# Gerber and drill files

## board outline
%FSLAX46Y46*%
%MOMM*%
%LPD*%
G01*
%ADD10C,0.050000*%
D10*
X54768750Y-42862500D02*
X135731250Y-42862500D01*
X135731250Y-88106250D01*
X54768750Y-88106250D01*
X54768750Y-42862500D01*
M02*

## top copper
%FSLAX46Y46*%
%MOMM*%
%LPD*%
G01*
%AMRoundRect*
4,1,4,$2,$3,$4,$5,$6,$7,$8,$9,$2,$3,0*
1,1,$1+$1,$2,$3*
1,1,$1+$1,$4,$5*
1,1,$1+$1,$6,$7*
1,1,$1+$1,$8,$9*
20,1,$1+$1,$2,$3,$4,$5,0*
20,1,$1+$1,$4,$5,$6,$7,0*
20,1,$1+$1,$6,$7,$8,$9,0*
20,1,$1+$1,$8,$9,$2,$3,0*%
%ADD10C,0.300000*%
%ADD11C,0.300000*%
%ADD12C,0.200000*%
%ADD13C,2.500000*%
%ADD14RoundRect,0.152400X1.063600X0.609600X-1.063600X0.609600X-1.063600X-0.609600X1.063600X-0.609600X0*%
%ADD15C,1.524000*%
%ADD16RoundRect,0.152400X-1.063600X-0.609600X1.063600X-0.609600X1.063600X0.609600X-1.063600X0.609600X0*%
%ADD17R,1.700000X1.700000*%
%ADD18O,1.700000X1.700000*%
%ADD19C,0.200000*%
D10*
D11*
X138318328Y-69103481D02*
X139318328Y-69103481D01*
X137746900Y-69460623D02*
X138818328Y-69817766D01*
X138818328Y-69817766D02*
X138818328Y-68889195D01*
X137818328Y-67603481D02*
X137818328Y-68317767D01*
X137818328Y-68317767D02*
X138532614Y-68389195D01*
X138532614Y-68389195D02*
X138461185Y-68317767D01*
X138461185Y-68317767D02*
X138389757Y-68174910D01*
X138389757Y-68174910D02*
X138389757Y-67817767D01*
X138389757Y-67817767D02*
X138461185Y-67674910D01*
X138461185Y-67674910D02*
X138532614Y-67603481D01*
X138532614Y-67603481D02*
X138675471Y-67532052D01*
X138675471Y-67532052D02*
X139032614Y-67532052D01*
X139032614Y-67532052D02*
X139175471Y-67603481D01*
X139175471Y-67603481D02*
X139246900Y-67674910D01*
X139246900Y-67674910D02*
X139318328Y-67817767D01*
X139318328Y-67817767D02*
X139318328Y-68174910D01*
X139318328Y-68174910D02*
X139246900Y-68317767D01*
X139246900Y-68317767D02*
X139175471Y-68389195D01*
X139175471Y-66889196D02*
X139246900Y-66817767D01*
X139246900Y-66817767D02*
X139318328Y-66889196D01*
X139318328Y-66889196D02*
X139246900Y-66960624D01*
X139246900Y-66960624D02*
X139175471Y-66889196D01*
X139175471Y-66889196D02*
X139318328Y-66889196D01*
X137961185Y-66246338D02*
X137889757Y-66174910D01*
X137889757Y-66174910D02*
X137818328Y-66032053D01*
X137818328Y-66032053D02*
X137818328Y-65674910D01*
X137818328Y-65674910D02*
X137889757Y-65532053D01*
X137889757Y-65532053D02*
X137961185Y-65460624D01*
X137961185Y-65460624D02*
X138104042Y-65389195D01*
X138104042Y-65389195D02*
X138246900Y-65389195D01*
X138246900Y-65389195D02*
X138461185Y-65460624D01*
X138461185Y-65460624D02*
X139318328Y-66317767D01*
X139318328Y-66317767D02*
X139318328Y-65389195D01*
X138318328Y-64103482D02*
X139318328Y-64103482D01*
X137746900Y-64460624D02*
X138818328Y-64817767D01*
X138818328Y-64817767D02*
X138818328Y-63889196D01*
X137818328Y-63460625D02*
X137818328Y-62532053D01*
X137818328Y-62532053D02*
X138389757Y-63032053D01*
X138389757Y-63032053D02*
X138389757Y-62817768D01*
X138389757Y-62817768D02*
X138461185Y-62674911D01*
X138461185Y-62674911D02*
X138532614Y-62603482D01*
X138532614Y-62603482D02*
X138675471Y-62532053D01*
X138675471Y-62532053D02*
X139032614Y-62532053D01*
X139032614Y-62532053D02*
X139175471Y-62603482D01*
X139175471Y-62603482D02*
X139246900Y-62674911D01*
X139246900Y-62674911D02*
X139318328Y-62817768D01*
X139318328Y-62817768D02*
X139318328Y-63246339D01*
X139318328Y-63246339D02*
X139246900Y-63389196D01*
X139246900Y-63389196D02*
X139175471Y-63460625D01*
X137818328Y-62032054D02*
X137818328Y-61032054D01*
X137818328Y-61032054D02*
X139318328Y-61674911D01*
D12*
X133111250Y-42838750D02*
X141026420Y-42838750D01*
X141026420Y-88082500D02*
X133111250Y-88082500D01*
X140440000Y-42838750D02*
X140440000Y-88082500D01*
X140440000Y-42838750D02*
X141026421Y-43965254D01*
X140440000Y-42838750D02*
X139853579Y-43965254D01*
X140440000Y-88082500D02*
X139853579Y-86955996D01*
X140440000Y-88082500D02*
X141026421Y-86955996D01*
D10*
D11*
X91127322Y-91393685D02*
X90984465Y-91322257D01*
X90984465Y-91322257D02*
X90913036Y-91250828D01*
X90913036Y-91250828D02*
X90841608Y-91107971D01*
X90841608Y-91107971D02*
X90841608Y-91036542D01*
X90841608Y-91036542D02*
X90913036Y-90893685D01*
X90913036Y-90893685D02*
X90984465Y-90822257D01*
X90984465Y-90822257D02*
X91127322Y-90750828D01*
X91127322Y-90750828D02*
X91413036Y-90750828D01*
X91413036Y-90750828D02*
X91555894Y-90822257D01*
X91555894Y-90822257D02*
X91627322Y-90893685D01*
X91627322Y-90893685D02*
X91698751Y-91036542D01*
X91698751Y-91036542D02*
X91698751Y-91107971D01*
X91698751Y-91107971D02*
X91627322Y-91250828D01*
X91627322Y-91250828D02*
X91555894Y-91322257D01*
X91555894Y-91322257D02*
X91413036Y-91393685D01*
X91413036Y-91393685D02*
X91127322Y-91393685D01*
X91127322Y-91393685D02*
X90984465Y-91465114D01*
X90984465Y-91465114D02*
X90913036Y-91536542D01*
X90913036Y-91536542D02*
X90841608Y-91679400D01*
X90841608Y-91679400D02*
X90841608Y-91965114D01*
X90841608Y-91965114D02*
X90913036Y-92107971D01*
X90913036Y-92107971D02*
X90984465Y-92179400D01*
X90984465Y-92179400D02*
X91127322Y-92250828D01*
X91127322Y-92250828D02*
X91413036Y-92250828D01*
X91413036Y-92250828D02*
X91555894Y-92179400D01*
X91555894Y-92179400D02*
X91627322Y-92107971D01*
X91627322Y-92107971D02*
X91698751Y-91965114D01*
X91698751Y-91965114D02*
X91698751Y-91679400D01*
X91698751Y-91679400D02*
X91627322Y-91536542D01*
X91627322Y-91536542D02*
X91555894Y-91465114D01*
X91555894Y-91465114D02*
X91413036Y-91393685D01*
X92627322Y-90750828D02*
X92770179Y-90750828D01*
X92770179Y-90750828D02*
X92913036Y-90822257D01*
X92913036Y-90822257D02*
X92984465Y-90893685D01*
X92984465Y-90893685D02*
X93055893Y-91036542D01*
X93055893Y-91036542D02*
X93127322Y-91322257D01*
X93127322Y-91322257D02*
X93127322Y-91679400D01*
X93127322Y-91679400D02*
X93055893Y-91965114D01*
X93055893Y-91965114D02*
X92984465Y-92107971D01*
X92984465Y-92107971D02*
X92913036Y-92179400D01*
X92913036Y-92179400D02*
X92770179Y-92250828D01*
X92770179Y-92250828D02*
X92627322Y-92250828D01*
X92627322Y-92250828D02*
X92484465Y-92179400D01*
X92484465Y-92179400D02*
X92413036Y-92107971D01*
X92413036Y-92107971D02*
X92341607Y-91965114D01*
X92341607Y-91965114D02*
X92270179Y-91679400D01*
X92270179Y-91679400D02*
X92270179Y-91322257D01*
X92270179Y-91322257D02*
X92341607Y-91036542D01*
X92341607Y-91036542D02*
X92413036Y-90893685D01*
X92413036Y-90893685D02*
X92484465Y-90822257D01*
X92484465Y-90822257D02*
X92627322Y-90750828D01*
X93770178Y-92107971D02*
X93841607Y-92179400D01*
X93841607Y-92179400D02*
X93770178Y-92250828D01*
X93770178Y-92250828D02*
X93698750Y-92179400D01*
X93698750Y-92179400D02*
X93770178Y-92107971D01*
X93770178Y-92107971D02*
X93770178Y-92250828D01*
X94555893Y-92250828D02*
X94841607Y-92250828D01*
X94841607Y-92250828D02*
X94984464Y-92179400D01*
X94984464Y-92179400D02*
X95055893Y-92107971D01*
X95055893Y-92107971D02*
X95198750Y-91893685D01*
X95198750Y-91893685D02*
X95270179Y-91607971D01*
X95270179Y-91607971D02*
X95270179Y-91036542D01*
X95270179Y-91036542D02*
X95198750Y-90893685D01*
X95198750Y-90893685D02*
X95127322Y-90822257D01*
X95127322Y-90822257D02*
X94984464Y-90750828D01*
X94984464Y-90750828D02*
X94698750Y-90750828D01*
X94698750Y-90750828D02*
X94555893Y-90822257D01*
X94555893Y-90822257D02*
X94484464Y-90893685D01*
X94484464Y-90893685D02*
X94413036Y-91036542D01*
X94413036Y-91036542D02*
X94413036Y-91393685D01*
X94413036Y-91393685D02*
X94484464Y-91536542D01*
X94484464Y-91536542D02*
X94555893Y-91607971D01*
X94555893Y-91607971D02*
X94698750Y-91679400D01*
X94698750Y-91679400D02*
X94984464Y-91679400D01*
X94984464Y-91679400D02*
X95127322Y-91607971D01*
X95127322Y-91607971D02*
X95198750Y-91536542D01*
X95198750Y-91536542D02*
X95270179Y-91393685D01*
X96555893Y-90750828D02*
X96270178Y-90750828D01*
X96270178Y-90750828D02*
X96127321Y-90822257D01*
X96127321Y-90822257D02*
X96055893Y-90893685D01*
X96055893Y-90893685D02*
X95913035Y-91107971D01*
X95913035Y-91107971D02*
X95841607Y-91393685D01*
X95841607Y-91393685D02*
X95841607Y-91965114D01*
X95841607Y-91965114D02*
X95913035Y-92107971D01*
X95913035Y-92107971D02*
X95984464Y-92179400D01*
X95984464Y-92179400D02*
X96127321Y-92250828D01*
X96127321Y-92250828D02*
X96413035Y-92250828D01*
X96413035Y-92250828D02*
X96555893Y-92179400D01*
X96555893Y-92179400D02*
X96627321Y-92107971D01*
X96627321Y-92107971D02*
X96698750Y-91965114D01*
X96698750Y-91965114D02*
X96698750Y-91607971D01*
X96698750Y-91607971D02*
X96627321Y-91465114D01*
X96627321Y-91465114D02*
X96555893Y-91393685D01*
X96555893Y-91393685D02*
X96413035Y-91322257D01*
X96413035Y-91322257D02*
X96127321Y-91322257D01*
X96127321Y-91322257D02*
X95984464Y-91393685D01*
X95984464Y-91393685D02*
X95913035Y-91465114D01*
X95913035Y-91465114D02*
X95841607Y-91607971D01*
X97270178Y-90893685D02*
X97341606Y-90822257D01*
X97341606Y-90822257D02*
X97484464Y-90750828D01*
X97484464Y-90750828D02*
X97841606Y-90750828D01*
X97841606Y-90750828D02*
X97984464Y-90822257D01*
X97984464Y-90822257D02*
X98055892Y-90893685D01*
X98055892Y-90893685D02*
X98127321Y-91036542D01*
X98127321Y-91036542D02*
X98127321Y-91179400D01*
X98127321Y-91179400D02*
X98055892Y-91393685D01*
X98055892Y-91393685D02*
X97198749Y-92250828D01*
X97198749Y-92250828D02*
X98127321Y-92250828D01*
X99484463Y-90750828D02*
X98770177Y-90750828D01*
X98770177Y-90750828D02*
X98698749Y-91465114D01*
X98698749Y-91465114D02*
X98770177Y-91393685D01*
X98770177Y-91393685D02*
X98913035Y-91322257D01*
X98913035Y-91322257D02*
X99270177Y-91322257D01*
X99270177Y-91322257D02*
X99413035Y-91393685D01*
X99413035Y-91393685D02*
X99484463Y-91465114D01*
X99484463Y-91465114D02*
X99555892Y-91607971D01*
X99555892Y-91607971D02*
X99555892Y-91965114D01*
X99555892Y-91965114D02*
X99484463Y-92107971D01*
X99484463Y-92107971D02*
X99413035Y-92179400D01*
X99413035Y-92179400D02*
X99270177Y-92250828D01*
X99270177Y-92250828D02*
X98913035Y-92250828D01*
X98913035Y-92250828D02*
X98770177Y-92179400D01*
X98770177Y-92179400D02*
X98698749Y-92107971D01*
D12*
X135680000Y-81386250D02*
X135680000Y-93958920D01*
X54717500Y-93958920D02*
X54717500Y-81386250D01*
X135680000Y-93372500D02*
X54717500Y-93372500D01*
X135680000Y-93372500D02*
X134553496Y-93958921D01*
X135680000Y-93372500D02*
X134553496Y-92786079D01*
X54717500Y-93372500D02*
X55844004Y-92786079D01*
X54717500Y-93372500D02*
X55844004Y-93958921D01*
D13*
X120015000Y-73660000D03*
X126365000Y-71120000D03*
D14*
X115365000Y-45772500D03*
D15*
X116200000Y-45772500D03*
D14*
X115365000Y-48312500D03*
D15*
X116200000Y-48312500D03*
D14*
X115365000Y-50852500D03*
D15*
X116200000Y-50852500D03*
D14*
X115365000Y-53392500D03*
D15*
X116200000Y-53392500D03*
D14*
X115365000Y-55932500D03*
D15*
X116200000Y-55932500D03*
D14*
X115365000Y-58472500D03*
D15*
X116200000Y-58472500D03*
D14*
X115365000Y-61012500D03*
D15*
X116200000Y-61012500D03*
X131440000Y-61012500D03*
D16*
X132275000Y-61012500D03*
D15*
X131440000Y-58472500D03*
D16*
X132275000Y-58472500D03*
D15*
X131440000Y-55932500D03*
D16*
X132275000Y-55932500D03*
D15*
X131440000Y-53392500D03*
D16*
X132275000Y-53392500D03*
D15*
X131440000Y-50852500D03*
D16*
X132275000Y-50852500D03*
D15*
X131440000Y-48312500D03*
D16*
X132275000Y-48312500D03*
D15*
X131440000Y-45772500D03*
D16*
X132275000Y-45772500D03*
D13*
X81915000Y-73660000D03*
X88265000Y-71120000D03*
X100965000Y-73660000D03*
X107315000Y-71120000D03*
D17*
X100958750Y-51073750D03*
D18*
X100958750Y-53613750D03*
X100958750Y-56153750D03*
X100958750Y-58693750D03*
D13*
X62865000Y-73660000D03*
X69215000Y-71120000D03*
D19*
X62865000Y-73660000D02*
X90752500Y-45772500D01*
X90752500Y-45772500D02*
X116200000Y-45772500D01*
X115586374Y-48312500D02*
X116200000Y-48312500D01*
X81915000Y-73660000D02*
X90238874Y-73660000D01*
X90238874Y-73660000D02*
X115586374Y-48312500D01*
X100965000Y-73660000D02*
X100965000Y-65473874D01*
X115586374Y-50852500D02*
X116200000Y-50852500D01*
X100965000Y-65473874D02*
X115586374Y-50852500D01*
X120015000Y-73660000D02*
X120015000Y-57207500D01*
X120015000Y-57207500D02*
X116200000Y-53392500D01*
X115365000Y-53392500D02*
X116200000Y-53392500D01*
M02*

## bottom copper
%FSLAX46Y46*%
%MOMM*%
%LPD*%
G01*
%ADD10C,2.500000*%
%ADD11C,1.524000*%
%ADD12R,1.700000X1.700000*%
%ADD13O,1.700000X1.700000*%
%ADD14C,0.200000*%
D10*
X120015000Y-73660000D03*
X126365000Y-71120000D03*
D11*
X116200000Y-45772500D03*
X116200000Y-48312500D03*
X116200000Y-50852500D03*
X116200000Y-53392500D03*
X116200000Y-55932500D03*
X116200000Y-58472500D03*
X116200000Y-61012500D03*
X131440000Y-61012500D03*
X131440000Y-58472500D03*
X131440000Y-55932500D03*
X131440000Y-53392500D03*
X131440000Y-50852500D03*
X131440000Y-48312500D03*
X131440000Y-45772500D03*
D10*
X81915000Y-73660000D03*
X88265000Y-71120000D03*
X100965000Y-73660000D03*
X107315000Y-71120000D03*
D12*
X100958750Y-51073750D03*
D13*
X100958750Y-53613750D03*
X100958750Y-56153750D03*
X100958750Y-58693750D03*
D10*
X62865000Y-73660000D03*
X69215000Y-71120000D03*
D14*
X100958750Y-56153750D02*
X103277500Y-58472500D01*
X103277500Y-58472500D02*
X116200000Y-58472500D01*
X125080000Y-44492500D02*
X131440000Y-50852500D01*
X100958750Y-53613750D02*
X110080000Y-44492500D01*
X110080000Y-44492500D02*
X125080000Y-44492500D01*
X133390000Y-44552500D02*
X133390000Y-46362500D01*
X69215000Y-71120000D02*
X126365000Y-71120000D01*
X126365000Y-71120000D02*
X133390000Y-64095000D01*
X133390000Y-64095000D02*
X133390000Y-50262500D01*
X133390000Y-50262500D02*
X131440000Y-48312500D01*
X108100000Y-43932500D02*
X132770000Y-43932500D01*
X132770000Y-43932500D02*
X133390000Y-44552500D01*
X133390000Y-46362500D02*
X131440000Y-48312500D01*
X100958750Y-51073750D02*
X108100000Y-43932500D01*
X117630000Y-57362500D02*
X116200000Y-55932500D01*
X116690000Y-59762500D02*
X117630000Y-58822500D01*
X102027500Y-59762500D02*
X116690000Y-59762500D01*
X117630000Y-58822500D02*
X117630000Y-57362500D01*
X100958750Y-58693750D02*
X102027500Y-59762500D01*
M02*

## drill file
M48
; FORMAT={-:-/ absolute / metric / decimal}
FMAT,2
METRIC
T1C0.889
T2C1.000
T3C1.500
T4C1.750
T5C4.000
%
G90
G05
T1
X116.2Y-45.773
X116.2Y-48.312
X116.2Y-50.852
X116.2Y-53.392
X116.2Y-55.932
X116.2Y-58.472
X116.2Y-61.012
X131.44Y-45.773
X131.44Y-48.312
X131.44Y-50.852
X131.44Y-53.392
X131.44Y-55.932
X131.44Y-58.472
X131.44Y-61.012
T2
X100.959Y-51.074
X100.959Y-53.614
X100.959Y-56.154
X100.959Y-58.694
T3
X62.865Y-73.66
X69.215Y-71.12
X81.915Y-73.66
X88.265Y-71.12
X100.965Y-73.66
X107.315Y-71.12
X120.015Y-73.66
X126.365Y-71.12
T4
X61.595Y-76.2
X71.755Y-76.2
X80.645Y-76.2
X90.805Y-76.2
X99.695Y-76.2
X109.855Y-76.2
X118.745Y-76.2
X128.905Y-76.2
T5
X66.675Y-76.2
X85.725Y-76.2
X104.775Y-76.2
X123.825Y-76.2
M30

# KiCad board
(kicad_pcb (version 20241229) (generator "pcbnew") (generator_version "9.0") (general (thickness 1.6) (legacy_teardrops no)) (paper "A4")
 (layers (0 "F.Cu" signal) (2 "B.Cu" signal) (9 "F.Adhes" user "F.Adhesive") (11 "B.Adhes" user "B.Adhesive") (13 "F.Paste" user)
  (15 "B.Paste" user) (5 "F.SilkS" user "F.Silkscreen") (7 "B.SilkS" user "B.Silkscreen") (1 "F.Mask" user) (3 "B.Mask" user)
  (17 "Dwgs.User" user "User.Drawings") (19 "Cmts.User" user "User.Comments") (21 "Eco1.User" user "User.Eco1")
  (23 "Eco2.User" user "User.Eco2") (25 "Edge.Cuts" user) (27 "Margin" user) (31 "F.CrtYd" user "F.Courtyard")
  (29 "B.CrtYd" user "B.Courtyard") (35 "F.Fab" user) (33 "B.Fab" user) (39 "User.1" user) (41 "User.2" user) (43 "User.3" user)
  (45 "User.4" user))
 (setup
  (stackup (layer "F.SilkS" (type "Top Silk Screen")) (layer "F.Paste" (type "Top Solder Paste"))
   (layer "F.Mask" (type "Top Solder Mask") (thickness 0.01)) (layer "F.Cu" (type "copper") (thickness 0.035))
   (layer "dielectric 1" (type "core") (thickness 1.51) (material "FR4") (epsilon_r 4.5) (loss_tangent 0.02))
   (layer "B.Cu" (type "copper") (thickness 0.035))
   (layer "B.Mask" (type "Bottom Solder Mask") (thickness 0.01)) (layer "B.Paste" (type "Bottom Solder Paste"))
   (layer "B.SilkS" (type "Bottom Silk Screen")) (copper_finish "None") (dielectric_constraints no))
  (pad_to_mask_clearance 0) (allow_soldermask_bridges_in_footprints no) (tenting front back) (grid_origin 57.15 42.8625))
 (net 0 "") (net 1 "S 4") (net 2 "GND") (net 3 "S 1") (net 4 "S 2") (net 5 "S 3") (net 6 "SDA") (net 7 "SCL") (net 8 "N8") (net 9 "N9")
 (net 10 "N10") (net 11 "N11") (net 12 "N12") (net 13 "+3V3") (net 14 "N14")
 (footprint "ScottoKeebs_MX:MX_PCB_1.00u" (layer "F.Cu") (at 123.825 76.2)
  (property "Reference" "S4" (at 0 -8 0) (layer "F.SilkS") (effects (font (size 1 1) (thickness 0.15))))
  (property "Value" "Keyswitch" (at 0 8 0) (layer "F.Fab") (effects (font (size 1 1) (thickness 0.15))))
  (pad "" np_thru_hole circle (at -5.08 0) (size 1.75 1.75) (drill 1.75) (layers "*.Cu" "*.Mask"))
  (pad "" np_thru_hole circle (at 0 0) (size 4 4) (drill 4) (layers "*.Cu" "*.Mask"))
  (pad "" np_thru_hole circle (at 5.08 0) (size 1.75 1.75) (drill 1.75) (layers "*.Cu" "*.Mask"))
  (pad "1" thru_hole circle (at -3.81 -2.54) (size 2.5 2.5) (drill 1.5) (layers "*.Cu" "*.Mask") (remove_unused_layers no) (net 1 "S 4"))
  (pad "2" thru_hole circle (at 2.54 -5.08) (size 2.5 2.5) (drill 1.5) (layers "*.Cu" "*.Mask") (remove_unused_layers no) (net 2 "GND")))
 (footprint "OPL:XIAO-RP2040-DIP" (layer "F.Cu") (at 123.82 53.3925)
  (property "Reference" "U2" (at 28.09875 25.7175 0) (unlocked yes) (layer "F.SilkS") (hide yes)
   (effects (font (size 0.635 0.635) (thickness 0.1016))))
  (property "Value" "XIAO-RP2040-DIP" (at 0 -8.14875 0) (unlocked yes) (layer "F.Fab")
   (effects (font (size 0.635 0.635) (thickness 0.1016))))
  (pad "1" smd roundrect (at -8.455 -7.62 180) (size 2.432 1.524) (layers "F.Cu" "F.Mask") (roundrect_rratio 0.1) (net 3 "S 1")
   (thermal_bridge_angle 45))
  (pad "1" thru_hole circle (at -7.62 -7.62 180) (size 1.524 1.524) (drill 0.889) (layers "*.Cu" "*.Mask") (remove_unused_layers no)
   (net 3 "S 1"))
  (pad "2" smd roundrect (at -8.455 -5.08 180) (size 2.432 1.524) (layers "F.Cu" "F.Mask") (roundrect_rratio 0.1) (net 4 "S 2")
   (thermal_bridge_angle 45))
  (pad "2" thru_hole circle (at -7.62 -5.08 180) (size 1.524 1.524) (drill 0.889) (layers "*.Cu" "*.Mask") (remove_unused_layers no)
   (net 4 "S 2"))
  (pad "3" smd roundrect (at -8.455 -2.54 180) (size 2.432 1.524) (layers "F.Cu" "F.Mask") (roundrect_rratio 0.1) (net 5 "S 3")
   (thermal_bridge_angle 45))
  (pad "3" thru_hole circle (at -7.62 -2.54 180) (size 1.524 1.524) (drill 0.889) (layers "*.Cu" "*.Mask") (remove_unused_layers no)
   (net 5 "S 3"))
  (pad "4" smd roundrect (at -8.455 0 180) (size 2.432 1.524) (layers "F.Cu" "F.Mask") (roundrect_rratio 0.1) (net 1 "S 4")
   (thermal_bridge_angle 45))
  (pad "4" thru_hole circle (at -7.62 0 180) (size 1.524 1.524) (drill 0.889) (layers "*.Cu" "*.Mask") (remove_unused_layers no)
   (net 1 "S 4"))
  (pad "5" smd roundrect (at -8.455 2.54 180) (size 2.432 1.524) (layers "F.Cu" "F.Mask") (roundrect_rratio 0.1) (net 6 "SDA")
   (thermal_bridge_angle 45))
  (pad "5" thru_hole circle (at -7.62 2.54 180) (size 1.524 1.524) (drill 0.889) (layers "*.Cu" "*.Mask") (remove_unused_layers no)
   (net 6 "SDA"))
  (pad "6" smd roundrect (at -8.455 5.08 180) (size 2.432 1.524) (layers "F.Cu" "F.Mask") (roundrect_rratio 0.1) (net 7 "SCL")
   (thermal_bridge_angle 45))
  (pad "6" thru_hole circle (at -7.62 5.08 180) (size 1.524 1.524) (drill 0.889) (layers "*.Cu" "*.Mask") (remove_unused_layers no)
   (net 7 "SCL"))
  (pad "7" smd roundrect (at -8.455 7.62 180) (size 2.432 1.524) (layers "F.Cu" "F.Mask") (roundrect_rratio 0.1) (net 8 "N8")
   (thermal_bridge_angle 45))
  (pad "7" thru_hole circle (at -7.62 7.62 180) (size 1.524 1.524) (drill 0.889) (layers "*.Cu" "*.Mask") (remove_unused_layers no)
   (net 8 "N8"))
  (pad "8" thru_hole circle (at 7.62 7.62) (size 1.524 1.524) (drill 0.889) (layers "*.Cu" "*.Mask") (remove_unused_layers no) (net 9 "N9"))
  (pad "8" smd roundrect (at 8.455 7.62) (size 2.432 1.524) (layers "F.Cu" "F.Mask") (roundrect_rratio 0.1) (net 9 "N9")
   (thermal_bridge_angle 45))
  (pad "9" thru_hole circle (at 7.62 5.08) (size 1.524 1.524) (drill 0.889) (layers "*.Cu" "*.Mask") (remove_unused_layers no)
   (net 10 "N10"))
  (pad "9" smd roundrect (at 8.455 5.08) (size 2.432 1.524) (layers "F.Cu" "F.Mask") (roundrect_rratio 0.1) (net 10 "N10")
   (thermal_bridge_angle 45))
  (pad "10" thru_hole circle (at 7.62 2.54) (size 1.524 1.524) (drill 0.889) (layers "*.Cu" "*.Mask") (remove_unused_layers no)
   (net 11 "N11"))
  (pad "10" smd roundrect (at 8.455 2.54) (size 2.432 1.524) (layers "F.Cu" "F.Mask") (roundrect_rratio 0.1) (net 11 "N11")
   (thermal_bridge_angle 45))
  (pad "11" thru_hole circle (at 7.62 0) (size 1.524 1.524) (drill 0.889) (layers "*.Cu" "*.Mask") (remove_unused_layers no) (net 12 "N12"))
  (pad "11" smd roundrect (at 8.455 0) (size 2.432 1.524) (layers "F.Cu" "F.Mask") (roundrect_rratio 0.1) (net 12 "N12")
   (thermal_bridge_angle 45))
  (pad "12" thru_hole circle (at 7.62 -2.54) (size 1.524 1.524) (drill 0.889) (layers "*.Cu" "*.Mask") (remove_unused_layers no)
   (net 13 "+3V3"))
  (pad "12" smd roundrect (at 8.455 -2.54) (size 2.432 1.524) (layers "F.Cu" "F.Mask") (roundrect_rratio 0.1) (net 13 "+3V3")
   (thermal_bridge_angle 45))
  (pad "13" thru_hole circle (at 7.62 -5.08) (size 1.524 1.524) (drill 0.889) (layers "*.Cu" "*.Mask") (remove_unused_layers no)
   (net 2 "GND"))
  (pad "13" smd roundrect (at 8.455 -5.08) (size 2.432 1.524) (layers "F.Cu" "F.Mask") (roundrect_rratio 0.1) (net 2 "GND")
   (thermal_bridge_angle 45))
  (pad "14" thru_hole circle (at 7.62 -7.62) (size 1.524 1.524) (drill 0.889) (layers "*.Cu" "*.Mask") (remove_unused_layers no)
   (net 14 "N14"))
  (pad "14" smd roundrect (at 8.455 -7.62) (size 2.432 1.524) (layers "F.Cu" "F.Mask") (roundrect_rratio 0.1) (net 14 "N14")
   (thermal_bridge_angle 45)))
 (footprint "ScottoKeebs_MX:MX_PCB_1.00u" (layer "F.Cu") (at 85.725 76.2)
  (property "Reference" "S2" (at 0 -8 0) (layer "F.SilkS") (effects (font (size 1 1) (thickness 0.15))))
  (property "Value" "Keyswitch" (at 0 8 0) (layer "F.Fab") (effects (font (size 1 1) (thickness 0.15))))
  (pad "" np_thru_hole circle (at -5.08 0) (size 1.75 1.75) (drill 1.75) (layers "*.Cu" "*.Mask"))
  (pad "" np_thru_hole circle (at 0 0) (size 4 4) (drill 4) (layers "*.Cu" "*.Mask"))
  (pad "" np_thru_hole circle (at 5.08 0) (size 1.75 1.75) (drill 1.75) (layers "*.Cu" "*.Mask"))
  (pad "1" thru_hole circle (at -3.81 -2.54) (size 2.5 2.5) (drill 1.5) (layers "*.Cu" "*.Mask") (remove_unused_layers no) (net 4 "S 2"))
  (pad "2" thru_hole circle (at 2.54 -5.08) (size 2.5 2.5) (drill 1.5) (layers "*.Cu" "*.Mask") (remove_unused_layers no) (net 2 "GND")))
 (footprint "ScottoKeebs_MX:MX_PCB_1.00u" (layer "F.Cu") (at 104.775 76.2)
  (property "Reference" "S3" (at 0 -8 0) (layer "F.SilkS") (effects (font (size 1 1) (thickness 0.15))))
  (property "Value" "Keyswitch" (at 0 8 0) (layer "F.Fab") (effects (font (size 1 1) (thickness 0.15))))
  (pad "" np_thru_hole circle (at -5.08 0) (size 1.75 1.75) (drill 1.75) (layers "*.Cu" "*.Mask"))
  (pad "" np_thru_hole circle (at 0 0) (size 4 4) (drill 4) (layers "*.Cu" "*.Mask"))
  (pad "" np_thru_hole circle (at 5.08 0) (size 1.75 1.75) (drill 1.75) (layers "*.Cu" "*.Mask"))
  (pad "1" thru_hole circle (at -3.81 -2.54) (size 2.5 2.5) (drill 1.5) (layers "*.Cu" "*.Mask") (remove_unused_layers no) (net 5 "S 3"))
  (pad "2" thru_hole circle (at 2.54 -5.08) (size 2.5 2.5) (drill 1.5) (layers "*.Cu" "*.Mask") (remove_unused_layers no) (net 2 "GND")))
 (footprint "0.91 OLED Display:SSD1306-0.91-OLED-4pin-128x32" (layer "F.Cu") (at 64.45875 48.88375)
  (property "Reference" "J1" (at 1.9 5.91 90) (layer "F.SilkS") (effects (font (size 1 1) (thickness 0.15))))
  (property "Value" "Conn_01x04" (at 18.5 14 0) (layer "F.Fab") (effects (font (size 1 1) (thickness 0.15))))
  (pad "1" thru_hole rect (at 36.5 2.19) (size 1.7 1.7) (drill 1) (layers "*.Cu" "*.Mask") (remove_unused_layers no) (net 2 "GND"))
  (pad "2" thru_hole oval (at 36.5 4.73) (size 1.7 1.7) (drill 1) (layers "*.Cu" "*.Mask") (remove_unused_layers no) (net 13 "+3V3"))
  (pad "3" thru_hole oval (at 36.5 7.27) (size 1.7 1.7) (drill 1) (layers "*.Cu" "*.Mask") (remove_unused_layers no) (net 7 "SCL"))
  (pad "4" thru_hole oval (at 36.5 9.81) (size 1.7 1.7) (drill 1) (layers "*.Cu" "*.Mask") (remove_unused_layers no) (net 6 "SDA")))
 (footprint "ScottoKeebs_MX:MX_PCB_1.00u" (layer "F.Cu") (at 66.675 76.2)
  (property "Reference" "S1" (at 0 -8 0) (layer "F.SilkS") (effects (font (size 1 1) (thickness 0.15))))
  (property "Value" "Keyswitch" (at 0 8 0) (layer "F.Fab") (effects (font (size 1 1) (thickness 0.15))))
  (pad "" np_thru_hole circle (at -5.08 0) (size 1.75 1.75) (drill 1.75) (layers "*.Cu" "*.Mask"))
  (pad "" np_thru_hole circle (at 0 0) (size 4 4) (drill 4) (layers "*.Cu" "*.Mask"))
  (pad "" np_thru_hole circle (at 5.08 0) (size 1.75 1.75) (drill 1.75) (layers "*.Cu" "*.Mask"))
  (pad "1" thru_hole circle (at -3.81 -2.54) (size 2.5 2.5) (drill 1.5) (layers "*.Cu" "*.Mask") (remove_unused_layers no) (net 3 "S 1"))
  (pad "2" thru_hole circle (at 2.54 -5.08) (size 2.5 2.5) (drill 1.5) (layers "*.Cu" "*.Mask") (remove_unused_layers no) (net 2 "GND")))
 (gr_rect (start 54.76875 42.8625) (end 135.73125 88.10625) (stroke (width 0.05) (type default)) (fill no) (layer "Edge.Cuts"))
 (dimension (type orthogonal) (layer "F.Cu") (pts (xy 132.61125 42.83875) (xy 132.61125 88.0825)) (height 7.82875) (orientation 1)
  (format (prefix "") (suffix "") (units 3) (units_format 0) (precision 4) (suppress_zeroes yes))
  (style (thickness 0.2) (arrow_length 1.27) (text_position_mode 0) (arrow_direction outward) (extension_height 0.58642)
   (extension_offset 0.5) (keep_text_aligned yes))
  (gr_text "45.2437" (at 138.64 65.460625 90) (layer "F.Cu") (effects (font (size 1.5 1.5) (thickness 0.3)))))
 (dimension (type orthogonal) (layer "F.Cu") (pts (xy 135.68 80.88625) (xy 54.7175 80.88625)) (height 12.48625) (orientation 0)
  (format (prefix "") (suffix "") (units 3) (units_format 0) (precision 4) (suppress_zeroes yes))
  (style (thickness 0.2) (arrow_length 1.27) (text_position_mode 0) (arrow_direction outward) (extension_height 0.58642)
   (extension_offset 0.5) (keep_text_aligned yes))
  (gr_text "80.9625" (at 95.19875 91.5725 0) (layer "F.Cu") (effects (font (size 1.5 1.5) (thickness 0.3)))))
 (segment (start 100.95875 56.15375) (end 103.2775 58.4725) (width 0.2) (layer "B.Cu") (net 7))
 (segment (start 103.2775 58.4725) (end 116.2 58.4725) (width 0.2) (layer "B.Cu") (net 7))
 (segment (start 125.08 44.4925) (end 131.44 50.8525) (width 0.2) (layer "B.Cu") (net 13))
 (segment (start 100.95875 53.61375) (end 110.08 44.4925) (width 0.2) (layer "B.Cu") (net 13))
 (segment (start 110.08 44.4925) (end 125.08 44.4925) (width 0.2) (layer "B.Cu") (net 13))
 (segment (start 133.39 44.5525) (end 133.39 46.3625) (width 0.2) (layer "B.Cu") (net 2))
 (segment (start 69.215 71.12) (end 126.365 71.12) (width 0.2) (layer "B.Cu") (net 2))
 (segment (start 126.365 71.12) (end 133.39 64.095) (width 0.2) (layer "B.Cu") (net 2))
 (segment (start 133.39 64.095) (end 133.39 50.2625) (width 0.2) (layer "B.Cu") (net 2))
 (segment (start 133.39 50.2625) (end 131.44 48.3125) (width 0.2) (layer "B.Cu") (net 2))
 (segment (start 108.1 43.9325) (end 132.77 43.9325) (width 0.2) (layer "B.Cu") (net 2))
 (segment (start 132.77 43.9325) (end 133.39 44.5525) (width 0.2) (layer "B.Cu") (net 2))
 (segment (start 133.39 46.3625) (end 131.44 48.3125) (width 0.2) (layer "B.Cu") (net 2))
 (segment (start 100.95875 51.07375) (end 108.1 43.9325) (width 0.2) (layer "B.Cu") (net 2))
 (segment (start 117.63 57.3625) (end 116.2 55.9325) (width 0.2) (layer "B.Cu") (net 6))
 (segment (start 116.69 59.7625) (end 117.63 58.8225) (width 0.2) (layer "B.Cu") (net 6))
 (segment (start 102.0275 59.7625) (end 116.69 59.7625) (width 0.2) (layer "B.Cu") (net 6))
 (segment (start 117.63 58.8225) (end 117.63 57.3625) (width 0.2) (layer "B.Cu") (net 6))
 (segment (start 100.95875 58.69375) (end 102.0275 59.7625) (width 0.2) (layer "B.Cu") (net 6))
 (segment (start 62.865 73.66) (end 90.7525 45.7725) (width 0.2) (layer "F.Cu") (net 3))
 (segment (start 90.7525 45.7725) (end 116.2 45.7725) (width 0.2) (layer "F.Cu") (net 3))
 (segment (start 115.586374 48.3125) (end 116.2 48.3125) (width 0.2) (layer "F.Cu") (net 4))
 (segment (start 81.915 73.66) (end 90.238874 73.66) (width 0.2) (layer "F.Cu") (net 4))
 (segment (start 90.238874 73.66) (end 115.586374 48.3125) (width 0.2) (layer "F.Cu") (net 4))
 (segment (start 100.965 73.66) (end 100.965 65.473874) (width 0.2) (layer "F.Cu") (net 5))
 (segment (start 115.586374 50.8525) (end 116.2 50.8525) (width 0.2) (layer "F.Cu") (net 5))
 (segment (start 100.965 65.473874) (end 115.586374 50.8525) (width 0.2) (layer "F.Cu") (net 5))
 (segment (start 120.015 73.66) (end 120.015 57.2075) (width 0.2) (layer "F.Cu") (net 1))
 (segment (start 120.015 57.2075) (end 116.2 53.3925) (width 0.2) (layer "F.Cu") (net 1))
 (segment (start 115.365 53.3925) (end 116.2 53.3925) (width 0.2) (layer "F.Cu") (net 1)))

